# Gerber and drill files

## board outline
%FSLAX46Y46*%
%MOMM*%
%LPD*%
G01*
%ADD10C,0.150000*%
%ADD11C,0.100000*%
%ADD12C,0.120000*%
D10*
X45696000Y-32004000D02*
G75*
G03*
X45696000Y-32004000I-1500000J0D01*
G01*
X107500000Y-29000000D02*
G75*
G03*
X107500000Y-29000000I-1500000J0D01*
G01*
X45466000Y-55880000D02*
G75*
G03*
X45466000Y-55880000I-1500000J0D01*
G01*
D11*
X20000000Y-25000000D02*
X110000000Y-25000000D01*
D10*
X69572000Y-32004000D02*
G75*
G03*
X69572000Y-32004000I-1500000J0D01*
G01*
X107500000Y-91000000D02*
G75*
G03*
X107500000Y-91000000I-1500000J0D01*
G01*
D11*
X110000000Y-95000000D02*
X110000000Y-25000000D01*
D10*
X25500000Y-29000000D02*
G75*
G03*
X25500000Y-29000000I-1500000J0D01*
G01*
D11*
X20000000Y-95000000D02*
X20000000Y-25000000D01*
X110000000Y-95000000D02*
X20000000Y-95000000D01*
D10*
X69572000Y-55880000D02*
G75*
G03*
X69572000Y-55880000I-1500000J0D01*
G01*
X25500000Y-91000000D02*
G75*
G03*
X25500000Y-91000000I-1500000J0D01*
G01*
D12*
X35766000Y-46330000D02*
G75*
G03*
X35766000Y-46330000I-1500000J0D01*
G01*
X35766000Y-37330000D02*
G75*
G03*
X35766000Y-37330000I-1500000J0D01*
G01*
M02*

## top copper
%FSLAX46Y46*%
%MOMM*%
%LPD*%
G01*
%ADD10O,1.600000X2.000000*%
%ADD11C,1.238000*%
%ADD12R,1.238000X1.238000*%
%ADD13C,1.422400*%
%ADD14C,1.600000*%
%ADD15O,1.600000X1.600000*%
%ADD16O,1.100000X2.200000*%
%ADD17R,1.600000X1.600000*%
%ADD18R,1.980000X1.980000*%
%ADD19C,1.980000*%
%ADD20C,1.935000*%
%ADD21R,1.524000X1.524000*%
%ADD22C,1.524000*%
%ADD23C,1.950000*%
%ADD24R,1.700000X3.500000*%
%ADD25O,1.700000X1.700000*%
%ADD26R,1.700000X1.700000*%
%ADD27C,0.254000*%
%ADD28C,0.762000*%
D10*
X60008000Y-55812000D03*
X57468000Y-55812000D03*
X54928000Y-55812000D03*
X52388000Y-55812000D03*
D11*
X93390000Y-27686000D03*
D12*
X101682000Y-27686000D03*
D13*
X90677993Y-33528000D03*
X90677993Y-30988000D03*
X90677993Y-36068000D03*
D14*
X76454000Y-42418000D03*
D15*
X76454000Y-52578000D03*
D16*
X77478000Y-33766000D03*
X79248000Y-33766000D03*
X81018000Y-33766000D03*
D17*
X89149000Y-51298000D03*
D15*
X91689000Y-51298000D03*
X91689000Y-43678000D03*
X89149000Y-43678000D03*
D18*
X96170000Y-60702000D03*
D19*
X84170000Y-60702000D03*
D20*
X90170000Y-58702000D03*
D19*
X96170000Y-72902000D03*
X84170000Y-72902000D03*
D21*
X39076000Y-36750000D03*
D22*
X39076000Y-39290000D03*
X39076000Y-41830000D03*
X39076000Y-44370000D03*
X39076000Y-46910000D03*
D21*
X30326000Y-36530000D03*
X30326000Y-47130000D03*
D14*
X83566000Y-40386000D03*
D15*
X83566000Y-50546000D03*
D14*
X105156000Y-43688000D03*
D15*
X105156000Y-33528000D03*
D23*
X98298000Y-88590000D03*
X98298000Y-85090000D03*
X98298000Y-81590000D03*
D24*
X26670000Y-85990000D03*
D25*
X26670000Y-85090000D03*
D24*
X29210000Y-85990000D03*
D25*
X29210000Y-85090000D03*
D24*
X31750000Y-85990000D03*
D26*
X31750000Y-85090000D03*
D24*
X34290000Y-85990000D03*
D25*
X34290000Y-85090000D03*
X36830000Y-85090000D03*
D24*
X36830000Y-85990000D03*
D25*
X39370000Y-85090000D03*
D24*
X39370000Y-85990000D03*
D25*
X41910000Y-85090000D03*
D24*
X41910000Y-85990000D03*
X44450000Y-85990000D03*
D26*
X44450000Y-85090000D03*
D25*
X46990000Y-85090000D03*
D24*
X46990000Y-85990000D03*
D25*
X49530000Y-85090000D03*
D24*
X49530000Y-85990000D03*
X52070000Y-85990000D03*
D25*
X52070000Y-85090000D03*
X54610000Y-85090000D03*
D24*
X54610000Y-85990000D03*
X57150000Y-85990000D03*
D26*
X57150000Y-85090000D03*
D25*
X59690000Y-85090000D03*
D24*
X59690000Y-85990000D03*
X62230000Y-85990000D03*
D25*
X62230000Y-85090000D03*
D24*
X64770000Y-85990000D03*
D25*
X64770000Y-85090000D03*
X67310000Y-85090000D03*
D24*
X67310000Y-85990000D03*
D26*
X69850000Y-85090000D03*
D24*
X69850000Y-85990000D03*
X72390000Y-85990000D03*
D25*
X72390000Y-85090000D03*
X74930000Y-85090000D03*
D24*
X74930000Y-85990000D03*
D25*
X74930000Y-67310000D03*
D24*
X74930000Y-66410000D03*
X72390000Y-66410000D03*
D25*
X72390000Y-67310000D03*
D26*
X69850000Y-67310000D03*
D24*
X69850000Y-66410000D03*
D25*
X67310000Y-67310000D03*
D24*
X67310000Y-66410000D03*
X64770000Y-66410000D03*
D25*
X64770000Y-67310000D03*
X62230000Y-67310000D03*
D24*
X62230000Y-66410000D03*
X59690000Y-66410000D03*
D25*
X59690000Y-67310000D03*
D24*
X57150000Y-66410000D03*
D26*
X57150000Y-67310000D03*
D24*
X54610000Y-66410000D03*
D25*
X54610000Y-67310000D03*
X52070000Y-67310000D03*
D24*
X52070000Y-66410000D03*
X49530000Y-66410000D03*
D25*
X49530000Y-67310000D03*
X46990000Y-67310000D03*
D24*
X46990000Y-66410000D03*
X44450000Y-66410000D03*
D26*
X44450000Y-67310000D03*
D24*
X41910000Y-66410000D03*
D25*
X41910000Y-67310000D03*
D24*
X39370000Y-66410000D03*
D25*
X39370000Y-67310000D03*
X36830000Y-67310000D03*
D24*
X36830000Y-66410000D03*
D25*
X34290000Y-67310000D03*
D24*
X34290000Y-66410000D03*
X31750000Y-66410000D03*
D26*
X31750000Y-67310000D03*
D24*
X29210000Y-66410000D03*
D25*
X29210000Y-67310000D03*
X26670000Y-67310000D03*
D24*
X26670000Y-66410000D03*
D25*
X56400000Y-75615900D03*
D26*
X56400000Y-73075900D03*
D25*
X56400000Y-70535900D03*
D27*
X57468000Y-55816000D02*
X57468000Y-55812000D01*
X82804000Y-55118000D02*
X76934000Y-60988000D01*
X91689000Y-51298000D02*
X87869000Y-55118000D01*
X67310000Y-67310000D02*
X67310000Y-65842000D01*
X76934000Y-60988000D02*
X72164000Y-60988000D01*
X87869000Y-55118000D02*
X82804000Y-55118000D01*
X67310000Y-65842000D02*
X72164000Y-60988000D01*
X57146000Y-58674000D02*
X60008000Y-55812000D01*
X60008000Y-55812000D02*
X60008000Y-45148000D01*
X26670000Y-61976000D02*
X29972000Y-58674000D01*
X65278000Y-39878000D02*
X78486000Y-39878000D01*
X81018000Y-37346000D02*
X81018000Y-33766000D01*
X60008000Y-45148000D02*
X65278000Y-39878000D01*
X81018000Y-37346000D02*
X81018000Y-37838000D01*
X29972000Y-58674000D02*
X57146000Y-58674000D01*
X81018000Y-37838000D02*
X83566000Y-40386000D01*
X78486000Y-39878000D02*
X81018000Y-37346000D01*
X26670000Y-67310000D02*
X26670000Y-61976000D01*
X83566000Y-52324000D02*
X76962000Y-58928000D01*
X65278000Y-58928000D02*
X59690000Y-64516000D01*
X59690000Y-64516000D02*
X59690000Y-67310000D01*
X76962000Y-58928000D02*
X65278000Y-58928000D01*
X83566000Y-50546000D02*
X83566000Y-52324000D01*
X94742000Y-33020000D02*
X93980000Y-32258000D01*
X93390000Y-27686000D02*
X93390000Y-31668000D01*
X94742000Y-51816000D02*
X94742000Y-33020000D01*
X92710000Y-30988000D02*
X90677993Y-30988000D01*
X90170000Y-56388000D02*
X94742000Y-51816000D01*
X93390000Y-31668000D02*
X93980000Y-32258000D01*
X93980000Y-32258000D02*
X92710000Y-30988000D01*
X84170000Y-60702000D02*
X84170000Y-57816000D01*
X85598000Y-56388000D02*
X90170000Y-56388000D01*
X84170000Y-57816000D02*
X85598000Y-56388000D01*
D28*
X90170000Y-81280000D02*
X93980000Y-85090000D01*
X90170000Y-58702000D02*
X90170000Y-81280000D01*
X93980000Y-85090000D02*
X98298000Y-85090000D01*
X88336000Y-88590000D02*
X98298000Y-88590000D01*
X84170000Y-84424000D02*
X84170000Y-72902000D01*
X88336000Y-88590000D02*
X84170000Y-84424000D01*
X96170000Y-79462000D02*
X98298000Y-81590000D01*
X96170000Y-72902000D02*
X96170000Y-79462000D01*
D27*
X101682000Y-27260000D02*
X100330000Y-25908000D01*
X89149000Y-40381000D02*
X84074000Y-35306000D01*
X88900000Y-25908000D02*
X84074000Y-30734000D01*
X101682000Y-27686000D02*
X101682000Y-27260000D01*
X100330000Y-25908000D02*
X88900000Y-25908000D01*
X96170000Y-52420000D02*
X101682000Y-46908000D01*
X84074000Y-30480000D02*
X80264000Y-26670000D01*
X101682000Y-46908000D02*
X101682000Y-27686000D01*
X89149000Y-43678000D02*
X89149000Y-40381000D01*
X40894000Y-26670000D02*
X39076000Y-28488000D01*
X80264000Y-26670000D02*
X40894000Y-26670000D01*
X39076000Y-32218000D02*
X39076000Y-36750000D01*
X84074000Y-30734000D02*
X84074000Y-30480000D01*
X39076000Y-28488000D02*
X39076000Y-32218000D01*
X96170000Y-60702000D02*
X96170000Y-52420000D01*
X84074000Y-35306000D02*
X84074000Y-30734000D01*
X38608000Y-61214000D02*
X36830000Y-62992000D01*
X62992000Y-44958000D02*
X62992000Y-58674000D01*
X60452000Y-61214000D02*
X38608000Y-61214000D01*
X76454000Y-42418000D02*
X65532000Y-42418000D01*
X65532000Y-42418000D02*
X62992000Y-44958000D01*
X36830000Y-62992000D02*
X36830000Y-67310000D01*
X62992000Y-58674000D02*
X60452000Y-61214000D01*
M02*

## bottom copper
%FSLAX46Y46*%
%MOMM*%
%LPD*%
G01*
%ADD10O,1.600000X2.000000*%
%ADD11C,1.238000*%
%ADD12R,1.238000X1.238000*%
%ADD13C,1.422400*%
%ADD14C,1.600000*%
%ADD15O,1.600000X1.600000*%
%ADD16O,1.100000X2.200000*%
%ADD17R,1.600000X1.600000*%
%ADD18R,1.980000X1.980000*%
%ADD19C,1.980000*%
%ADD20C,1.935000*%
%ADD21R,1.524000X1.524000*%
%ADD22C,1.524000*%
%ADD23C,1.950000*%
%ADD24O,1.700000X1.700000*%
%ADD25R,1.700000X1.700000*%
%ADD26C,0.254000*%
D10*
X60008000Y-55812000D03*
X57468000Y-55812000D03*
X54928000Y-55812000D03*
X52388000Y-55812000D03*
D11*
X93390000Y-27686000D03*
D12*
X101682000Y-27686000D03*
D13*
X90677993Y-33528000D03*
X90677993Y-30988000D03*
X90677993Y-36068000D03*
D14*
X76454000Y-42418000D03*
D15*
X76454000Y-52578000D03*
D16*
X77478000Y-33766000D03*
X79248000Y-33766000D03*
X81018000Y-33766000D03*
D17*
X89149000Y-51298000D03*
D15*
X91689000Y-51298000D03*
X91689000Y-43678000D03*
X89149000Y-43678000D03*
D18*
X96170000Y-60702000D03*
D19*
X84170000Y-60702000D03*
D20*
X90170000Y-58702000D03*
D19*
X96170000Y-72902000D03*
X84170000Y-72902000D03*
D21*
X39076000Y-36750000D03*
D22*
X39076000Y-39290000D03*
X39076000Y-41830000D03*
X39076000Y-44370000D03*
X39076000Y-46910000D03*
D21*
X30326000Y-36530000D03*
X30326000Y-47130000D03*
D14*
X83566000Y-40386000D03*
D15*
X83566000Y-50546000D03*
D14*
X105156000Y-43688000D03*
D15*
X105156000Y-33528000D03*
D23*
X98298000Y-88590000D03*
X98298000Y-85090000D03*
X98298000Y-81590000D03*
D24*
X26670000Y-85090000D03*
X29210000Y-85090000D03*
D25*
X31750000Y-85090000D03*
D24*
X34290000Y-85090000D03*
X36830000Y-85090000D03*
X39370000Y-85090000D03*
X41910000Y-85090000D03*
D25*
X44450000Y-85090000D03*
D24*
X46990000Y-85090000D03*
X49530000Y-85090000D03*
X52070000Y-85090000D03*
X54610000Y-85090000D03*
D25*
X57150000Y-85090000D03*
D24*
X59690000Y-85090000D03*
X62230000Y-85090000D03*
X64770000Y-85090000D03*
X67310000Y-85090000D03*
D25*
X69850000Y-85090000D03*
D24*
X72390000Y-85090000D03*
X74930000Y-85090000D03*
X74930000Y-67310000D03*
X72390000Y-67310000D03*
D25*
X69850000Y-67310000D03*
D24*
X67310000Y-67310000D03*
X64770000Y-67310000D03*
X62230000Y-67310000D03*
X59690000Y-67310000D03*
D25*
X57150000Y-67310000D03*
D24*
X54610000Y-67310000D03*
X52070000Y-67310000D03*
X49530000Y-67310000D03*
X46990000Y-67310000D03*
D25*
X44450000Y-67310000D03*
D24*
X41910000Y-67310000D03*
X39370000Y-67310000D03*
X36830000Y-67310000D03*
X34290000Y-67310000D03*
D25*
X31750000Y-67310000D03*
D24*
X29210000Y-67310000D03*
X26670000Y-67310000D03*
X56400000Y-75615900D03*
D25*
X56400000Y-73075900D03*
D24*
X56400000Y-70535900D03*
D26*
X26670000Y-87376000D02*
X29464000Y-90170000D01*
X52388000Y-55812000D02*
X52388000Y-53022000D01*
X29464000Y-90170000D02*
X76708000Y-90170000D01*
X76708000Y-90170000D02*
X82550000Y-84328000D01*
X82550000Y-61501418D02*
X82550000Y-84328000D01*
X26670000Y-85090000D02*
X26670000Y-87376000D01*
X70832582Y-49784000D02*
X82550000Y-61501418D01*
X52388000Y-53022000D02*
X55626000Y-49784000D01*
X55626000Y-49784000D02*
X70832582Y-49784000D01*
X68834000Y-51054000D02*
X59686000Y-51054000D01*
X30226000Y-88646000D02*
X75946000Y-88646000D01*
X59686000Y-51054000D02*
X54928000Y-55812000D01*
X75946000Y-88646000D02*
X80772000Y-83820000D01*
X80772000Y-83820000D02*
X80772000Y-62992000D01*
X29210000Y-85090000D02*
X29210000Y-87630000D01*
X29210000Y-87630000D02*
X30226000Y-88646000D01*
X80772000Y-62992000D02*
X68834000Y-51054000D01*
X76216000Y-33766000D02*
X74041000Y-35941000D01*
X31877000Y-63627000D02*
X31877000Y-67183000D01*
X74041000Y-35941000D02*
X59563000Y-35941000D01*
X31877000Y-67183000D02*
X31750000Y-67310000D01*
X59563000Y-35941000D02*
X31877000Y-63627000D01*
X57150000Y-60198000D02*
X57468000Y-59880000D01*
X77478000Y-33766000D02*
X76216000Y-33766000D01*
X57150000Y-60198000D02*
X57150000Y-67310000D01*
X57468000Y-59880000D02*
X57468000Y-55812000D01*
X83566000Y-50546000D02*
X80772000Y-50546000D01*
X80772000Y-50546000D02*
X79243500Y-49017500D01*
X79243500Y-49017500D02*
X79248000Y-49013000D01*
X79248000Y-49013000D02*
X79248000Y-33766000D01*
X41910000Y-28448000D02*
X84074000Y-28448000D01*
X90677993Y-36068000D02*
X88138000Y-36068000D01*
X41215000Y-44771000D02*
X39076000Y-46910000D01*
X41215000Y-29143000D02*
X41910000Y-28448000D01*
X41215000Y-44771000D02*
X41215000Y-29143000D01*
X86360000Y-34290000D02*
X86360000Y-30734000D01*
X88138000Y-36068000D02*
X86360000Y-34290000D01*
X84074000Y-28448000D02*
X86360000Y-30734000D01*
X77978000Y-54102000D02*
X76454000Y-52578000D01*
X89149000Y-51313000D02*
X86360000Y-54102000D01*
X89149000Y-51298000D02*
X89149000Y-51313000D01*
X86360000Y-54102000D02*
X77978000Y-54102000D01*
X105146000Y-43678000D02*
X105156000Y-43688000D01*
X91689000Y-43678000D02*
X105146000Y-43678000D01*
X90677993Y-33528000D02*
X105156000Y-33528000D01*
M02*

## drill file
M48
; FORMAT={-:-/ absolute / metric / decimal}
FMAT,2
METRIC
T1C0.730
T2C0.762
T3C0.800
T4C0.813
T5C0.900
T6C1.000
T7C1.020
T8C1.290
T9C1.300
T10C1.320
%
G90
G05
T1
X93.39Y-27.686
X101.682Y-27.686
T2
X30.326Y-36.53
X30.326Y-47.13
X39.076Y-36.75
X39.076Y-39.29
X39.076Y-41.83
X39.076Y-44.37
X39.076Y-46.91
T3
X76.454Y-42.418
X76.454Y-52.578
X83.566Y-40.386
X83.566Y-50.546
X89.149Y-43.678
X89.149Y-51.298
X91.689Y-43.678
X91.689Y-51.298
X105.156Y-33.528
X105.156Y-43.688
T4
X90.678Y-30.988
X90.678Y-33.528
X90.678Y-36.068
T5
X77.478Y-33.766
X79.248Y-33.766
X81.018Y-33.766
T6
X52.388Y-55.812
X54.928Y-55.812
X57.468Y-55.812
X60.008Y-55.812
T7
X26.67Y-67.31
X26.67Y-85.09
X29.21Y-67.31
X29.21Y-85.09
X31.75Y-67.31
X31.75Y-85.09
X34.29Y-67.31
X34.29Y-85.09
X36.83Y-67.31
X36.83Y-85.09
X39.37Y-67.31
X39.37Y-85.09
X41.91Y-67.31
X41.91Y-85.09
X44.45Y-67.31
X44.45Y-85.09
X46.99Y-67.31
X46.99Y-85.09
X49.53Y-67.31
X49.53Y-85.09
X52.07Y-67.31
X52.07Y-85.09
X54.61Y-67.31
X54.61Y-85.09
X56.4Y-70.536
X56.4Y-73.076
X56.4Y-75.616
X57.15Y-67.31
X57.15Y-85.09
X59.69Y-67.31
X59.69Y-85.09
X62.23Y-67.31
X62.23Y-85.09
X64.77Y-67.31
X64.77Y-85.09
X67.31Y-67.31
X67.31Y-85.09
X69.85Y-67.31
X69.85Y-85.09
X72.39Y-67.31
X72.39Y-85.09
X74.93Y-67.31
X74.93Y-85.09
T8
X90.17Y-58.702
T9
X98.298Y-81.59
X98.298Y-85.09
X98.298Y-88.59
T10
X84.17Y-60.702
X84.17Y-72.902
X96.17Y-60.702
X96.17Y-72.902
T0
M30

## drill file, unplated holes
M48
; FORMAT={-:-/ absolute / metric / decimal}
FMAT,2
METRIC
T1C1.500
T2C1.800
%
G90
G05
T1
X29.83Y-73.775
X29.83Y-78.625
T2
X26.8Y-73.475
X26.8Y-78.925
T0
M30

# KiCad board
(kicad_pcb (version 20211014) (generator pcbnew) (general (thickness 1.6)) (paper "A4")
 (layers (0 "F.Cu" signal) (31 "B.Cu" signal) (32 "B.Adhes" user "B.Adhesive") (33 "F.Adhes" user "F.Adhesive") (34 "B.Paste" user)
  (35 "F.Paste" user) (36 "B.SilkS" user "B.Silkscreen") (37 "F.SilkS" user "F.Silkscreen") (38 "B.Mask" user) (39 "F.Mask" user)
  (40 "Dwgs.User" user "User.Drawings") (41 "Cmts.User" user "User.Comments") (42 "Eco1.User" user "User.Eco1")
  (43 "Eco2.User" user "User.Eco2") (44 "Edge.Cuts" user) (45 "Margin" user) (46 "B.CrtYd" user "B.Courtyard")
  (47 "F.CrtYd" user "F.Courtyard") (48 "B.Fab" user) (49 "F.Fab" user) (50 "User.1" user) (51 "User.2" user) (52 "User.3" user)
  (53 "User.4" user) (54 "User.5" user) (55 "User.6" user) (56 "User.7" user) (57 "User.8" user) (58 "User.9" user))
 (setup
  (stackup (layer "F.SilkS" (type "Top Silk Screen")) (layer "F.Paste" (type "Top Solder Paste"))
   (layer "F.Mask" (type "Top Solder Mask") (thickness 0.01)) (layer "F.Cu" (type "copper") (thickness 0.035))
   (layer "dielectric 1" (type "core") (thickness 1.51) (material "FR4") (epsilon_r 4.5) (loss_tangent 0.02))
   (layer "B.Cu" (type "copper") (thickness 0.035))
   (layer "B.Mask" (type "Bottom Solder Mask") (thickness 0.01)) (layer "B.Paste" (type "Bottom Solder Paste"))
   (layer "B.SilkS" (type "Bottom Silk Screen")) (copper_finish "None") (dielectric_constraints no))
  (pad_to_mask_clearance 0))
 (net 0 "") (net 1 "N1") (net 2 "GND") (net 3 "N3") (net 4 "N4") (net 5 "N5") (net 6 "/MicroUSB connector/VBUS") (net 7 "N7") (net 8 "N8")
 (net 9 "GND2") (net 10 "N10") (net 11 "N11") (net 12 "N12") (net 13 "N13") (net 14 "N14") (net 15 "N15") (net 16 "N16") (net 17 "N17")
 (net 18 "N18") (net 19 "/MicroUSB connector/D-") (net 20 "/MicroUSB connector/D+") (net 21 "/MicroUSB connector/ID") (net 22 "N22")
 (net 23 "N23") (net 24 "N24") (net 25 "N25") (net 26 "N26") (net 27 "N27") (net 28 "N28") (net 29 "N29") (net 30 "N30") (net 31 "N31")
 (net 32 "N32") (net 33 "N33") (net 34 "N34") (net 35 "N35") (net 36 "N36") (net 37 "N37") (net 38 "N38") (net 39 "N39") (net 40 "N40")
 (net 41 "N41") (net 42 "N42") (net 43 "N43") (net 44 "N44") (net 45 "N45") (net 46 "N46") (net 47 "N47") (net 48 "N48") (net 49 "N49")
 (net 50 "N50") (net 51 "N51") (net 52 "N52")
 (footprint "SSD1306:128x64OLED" (layer "F.Cu") (at 56.388 45.212 180)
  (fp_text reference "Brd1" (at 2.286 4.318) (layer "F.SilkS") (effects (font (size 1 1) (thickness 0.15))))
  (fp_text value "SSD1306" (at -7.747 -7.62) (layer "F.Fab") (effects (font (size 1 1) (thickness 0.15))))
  (pad "1" thru_hole oval locked (at -3.62 -10.6 270) (size 2 1.6) (drill 1) (layers *.Cu *.Mask) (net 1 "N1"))
  (pad "2" thru_hole oval locked (at -1.08 -10.6 270) (size 2 1.6) (drill 1) (layers *.Cu *.Mask) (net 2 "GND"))
  (pad "3" thru_hole oval locked (at 1.46 -10.6 270) (size 2 1.6) (drill 1) (layers *.Cu *.Mask) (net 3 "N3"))
  (pad "4" thru_hole oval locked (at 4 -10.6 270) (size 2 1.6) (drill 1) (layers *.Cu *.Mask) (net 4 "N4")))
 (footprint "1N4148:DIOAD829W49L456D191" (layer "F.Cu") (at 97.536 27.686 180)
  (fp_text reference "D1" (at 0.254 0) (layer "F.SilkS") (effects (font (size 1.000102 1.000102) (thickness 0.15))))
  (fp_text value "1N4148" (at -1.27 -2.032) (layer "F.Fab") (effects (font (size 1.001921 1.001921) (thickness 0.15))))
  (pad "A" thru_hole circle locked (at 4.146 0 180) (size 1.238 1.238) (drill 0.73) (layers *.Cu *.Mask) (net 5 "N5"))
  (pad "C" thru_hole rect locked (at -4.146 0 180) (size 1.238 1.238) (drill 0.73) (layers *.Cu *.Mask) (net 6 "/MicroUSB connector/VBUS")))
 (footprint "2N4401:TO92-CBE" (layer "F.Cu") (at 90.677993 33.528 90)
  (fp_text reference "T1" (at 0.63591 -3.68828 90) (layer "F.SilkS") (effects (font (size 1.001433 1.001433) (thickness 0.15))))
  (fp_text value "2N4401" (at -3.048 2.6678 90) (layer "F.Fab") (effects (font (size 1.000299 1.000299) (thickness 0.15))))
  (pad "B" thru_hole circle locked (at 0 0 90) (size 1.4224 1.4224) (drill 0.8128) (layers *.Cu *.Mask) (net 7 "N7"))
  (pad "C" thru_hole circle locked (at 2.54 0 90) (size 1.4224 1.4224) (drill 0.8128) (layers *.Cu *.Mask) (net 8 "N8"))
  (pad "E" thru_hole circle locked (at -2.54 0 90) (size 1.4224 1.4224) (drill 0.8128) (layers *.Cu *.Mask) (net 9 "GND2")))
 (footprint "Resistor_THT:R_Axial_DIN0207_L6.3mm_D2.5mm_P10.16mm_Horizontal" (layer "F.Cu") (at 76.454 42.418 -90)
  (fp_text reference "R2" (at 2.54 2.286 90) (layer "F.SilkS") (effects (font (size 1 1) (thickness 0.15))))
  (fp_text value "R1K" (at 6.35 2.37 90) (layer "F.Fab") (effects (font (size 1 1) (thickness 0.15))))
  (pad "1" thru_hole circle (at 0 0 270) (size 1.6 1.6) (drill 0.8) (layers *.Cu *.Mask) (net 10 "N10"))
  (pad "2" thru_hole oval (at 10.16 0 270) (size 1.6 1.6) (drill 0.8) (layers *.Cu *.Mask) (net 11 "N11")))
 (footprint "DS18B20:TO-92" (layer "F.Cu") (at 79.248 32.766)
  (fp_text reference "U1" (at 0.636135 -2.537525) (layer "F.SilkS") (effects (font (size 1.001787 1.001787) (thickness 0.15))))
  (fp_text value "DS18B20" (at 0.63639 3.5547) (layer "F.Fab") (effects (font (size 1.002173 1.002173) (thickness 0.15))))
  (pad "1" thru_hole oval locked (at -1.77 1) (size 1.1 2.2) (drill 0.9) (layers *.Cu *.Mask) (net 2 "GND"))
  (pad "2" thru_hole oval locked (at 0 1) (size 1.1 2.2) (drill 0.9) (layers *.Cu *.Mask) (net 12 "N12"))
  (pad "3" thru_hole oval locked (at 1.77 1) (size 1.1 2.2) (drill 0.9) (layers *.Cu *.Mask) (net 1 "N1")))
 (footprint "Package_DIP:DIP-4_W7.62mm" (layer "F.Cu") (at 89.149 51.298 90)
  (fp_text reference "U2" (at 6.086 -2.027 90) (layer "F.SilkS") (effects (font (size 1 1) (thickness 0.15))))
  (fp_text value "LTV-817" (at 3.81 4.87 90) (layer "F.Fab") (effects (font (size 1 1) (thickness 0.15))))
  (pad "1" thru_hole rect (at 0 0 90) (size 1.6 1.6) (drill 0.8) (layers *.Cu *.Mask) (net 11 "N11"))
  (pad "2" thru_hole oval (at 0 2.54 90) (size 1.6 1.6) (drill 0.8) (layers *.Cu *.Mask) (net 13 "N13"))
  (pad "3" thru_hole oval (at 7.62 2.54 90) (size 1.6 1.6) (drill 0.8) (layers *.Cu *.Mask) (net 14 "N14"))
  (pad "4" thru_hole oval (at 7.62 0 90) (size 1.6 1.6) (drill 0.8) (layers *.Cu *.Mask) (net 6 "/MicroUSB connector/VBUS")))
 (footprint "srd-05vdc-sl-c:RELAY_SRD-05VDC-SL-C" (layer "F.Cu") (at 90.17 66.802 -90)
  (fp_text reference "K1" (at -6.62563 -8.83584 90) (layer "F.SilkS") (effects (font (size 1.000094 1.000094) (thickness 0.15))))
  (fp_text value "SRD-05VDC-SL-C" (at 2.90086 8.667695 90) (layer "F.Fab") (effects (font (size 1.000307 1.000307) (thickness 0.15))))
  (pad "A1" thru_hole rect locked (at -6.1 -6 270) (size 1.98 1.98) (drill 1.32) (layers *.Cu *.Mask) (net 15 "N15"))
  (pad "A2" thru_hole circle locked (at -6.1 6 270) (size 1.98 1.98) (drill 1.32) (layers *.Cu *.Mask) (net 8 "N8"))
  (pad "COM" thru_hole circle locked (at -8.1 0 270) (size 1.935 1.935) (drill 1.29) (layers *.Cu *.Mask) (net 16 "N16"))
  (pad "NC" thru_hole circle locked (at 6.1 -6 270) (size 1.98 1.98) (drill 1.32) (layers *.Cu *.Mask) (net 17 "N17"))
  (pad "NO" thru_hole circle locked (at 6.1 6 270) (size 1.98 1.98) (drill 1.32) (layers *.Cu *.Mask) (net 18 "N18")))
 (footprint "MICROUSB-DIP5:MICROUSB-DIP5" (layer "F.Cu") (at 32.766 41.83)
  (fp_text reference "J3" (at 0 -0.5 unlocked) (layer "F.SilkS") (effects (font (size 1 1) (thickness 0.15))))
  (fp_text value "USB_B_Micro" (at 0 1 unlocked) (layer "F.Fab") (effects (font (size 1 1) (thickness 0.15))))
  (fp_circle (center 1.5 4.5) (end 3 4.5) (layer "Edge.Cuts") (width 0.12) (fill none))
  (fp_circle (center 1.5 -4.5) (end 3 -4.5) (layer "Edge.Cuts") (width 0.12) (fill none))
  (pad "1" thru_hole rect (at 6.31 -5.08) (size 1.524 1.524) (drill 0.762) (layers *.Cu *.Mask) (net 6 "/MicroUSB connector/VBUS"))
  (pad "2" thru_hole circle (at 6.31 -2.54) (size 1.524 1.524) (drill 0.762) (layers *.Cu *.Mask) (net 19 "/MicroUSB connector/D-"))
  (pad "3" thru_hole circle (at 6.31 0) (size 1.524 1.524) (drill 0.762) (layers *.Cu *.Mask) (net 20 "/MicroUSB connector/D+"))
  (pad "4" thru_hole circle (at 6.31 2.54) (size 1.524 1.524) (drill 0.762) (layers *.Cu *.Mask) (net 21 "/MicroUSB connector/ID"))
  (pad "5" thru_hole circle (at 6.31 5.08) (size 1.524 1.524) (drill 0.762) (layers *.Cu *.Mask) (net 9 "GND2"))
  (pad "6" thru_hole rect (at -2.44 -5.3) (size 1.524 1.524) (drill 0.762) (layers *.Cu *.Mask) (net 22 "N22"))
  (pad "7" thru_hole rect (at -2.44 5.3) (size 1.524 1.524) (drill 0.762) (layers *.Cu *.Mask)))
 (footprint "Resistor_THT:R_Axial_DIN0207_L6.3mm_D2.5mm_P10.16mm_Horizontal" (layer "F.Cu") (at 83.566 40.386 -90)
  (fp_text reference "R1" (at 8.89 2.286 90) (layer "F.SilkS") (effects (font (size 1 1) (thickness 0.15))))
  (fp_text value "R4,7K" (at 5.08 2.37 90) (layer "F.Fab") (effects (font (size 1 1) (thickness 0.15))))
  (pad "1" thru_hole circle (at 0 0 270) (size 1.6 1.6) (drill 0.8) (layers *.Cu *.Mask) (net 1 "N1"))
  (pad "2" thru_hole oval (at 10.16 0 270) (size 1.6 1.6) (drill 0.8) (layers *.Cu *.Mask) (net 12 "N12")))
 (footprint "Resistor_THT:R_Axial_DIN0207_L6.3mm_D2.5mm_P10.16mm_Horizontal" (layer "F.Cu") (at 105.156 43.688 90)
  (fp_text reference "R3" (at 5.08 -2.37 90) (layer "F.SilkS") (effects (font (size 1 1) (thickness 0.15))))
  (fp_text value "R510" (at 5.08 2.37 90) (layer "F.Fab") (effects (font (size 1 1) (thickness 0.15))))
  (pad "1" thru_hole circle (at 0 0 90) (size 1.6 1.6) (drill 0.8) (layers *.Cu *.Mask) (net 14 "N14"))
  (pad "2" thru_hole oval (at 10.16 0 90) (size 1.6 1.6) (drill 0.8) (layers *.Cu *.Mask) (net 7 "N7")))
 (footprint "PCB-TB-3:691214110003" (layer "F.Cu") (at 98.298 85.09 90)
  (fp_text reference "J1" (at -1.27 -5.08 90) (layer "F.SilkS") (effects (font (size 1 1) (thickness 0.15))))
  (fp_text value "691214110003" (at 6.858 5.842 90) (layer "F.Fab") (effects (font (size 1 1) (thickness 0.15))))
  (pad "1" thru_hole circle locked (at -3.5 0 90) (size 1.95 1.95) (drill 1.3) (layers *.Cu *.Mask) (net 18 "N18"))
  (pad "2" thru_hole circle locked (at 0 0 90) (size 1.95 1.95) (drill 1.3) (layers *.Cu *.Mask) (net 16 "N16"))
  (pad "3" thru_hole circle locked (at 3.5 0 90) (size 1.95 1.95) (drill 1.3) (layers *.Cu *.Mask) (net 17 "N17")))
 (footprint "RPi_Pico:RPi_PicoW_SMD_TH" (layer "F.Cu") (at 50.8 76.2 90)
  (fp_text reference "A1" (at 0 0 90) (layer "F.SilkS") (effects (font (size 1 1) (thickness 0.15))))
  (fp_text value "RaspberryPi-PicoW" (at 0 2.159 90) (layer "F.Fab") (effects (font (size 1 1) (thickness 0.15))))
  (pad "" np_thru_hole oval (at -2.425 -20.97 90) (size 1.5 1.5) (drill 1.5) (layers *.Cu *.Mask))
  (pad "" np_thru_hole oval (at 2.725 -24 90) (size 1.8 1.8) (drill 1.8) (layers *.Cu *.Mask))
  (pad "" np_thru_hole oval (at 2.425 -20.97 90) (size 1.5 1.5) (drill 1.5) (layers *.Cu *.Mask))
  (pad "" np_thru_hole oval (at -2.725 -24 90) (size 1.8 1.8) (drill 1.8) (layers *.Cu *.Mask))
  (pad "1" smd rect (at -8.89 -24.13 90) (size 3.5 1.7) (drill (offset -0.9 0)) (layers "F.Cu" "F.Mask") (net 4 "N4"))
  (pad "1" thru_hole oval (at -8.89 -24.13 90) (size 1.7 1.7) (drill 1.02) (layers *.Cu *.Mask) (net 4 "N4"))
  (pad "2" smd rect (at -8.89 -21.59 90) (size 3.5 1.7) (drill (offset -0.9 0)) (layers "F.Cu" "F.Mask") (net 3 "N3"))
  (pad "2" thru_hole oval (at -8.89 -21.59 90) (size 1.7 1.7) (drill 1.02) (layers *.Cu *.Mask) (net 3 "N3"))
  (pad "3" smd rect (at -8.89 -19.05 90) (size 3.5 1.7) (drill (offset -0.9 0)) (layers "F.Cu" "F.Mask") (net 2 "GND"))
  (pad "3" thru_hole rect (at -8.89 -19.05 90) (size 1.7 1.7) (drill 1.02) (layers *.Cu *.Mask) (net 2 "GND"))
  (pad "4" smd rect (at -8.89 -16.51 90) (size 3.5 1.7) (drill (offset -0.9 0)) (layers "F.Cu" "F.Mask") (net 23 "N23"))
  (pad "4" thru_hole oval (at -8.89 -16.51 90) (size 1.7 1.7) (drill 1.02) (layers *.Cu *.Mask) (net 23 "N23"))
  (pad "5" thru_hole oval (at -8.89 -13.97 90) (size 1.7 1.7) (drill 1.02) (layers *.Cu *.Mask) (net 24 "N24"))
  (pad "5" smd rect (at -8.89 -13.97 90) (size 3.5 1.7) (drill (offset -0.9 0)) (layers "F.Cu" "F.Mask") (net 24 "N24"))
  (pad "6" thru_hole oval (at -8.89 -11.43 90) (size 1.7 1.7) (drill 1.02) (layers *.Cu *.Mask) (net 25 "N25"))
  (pad "6" smd rect (at -8.89 -11.43 90) (size 3.5 1.7) (drill (offset -0.9 0)) (layers "F.Cu" "F.Mask") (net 25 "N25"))
  (pad "7" thru_hole oval (at -8.89 -8.89 90) (size 1.7 1.7) (drill 1.02) (layers *.Cu *.Mask) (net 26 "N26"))
  (pad "7" smd rect (at -8.89 -8.89 90) (size 3.5 1.7) (drill (offset -0.9 0)) (layers "F.Cu" "F.Mask") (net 26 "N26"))
  (pad "8" smd rect (at -8.89 -6.35 90) (size 3.5 1.7) (drill (offset -0.9 0)) (layers "F.Cu" "F.Mask") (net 2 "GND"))
  (pad "8" thru_hole rect (at -8.89 -6.35 90) (size 1.7 1.7) (drill 1.02) (layers *.Cu *.Mask) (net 2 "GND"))
  (pad "9" thru_hole oval (at -8.89 -3.81 90) (size 1.7 1.7) (drill 1.02) (layers *.Cu *.Mask) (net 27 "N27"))
  (pad "9" smd rect (at -8.89 -3.81 90) (size 3.5 1.7) (drill (offset -0.9 0)) (layers "F.Cu" "F.Mask") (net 27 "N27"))
  (pad "10" thru_hole oval (at -8.89 -1.27 90) (size 1.7 1.7) (drill 1.02) (layers *.Cu *.Mask) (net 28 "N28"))
  (pad "10" smd rect (at -8.89 -1.27 90) (size 3.5 1.7) (drill (offset -0.9 0)) (layers "F.Cu" "F.Mask") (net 28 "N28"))
  (pad "11" smd rect (at -8.89 1.27 90) (size 3.5 1.7) (drill (offset -0.9 0)) (layers "F.Cu" "F.Mask") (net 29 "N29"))
  (pad "11" thru_hole oval (at -8.89 1.27 90) (size 1.7 1.7) (drill 1.02) (layers *.Cu *.Mask) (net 29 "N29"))
  (pad "12" thru_hole oval (at -8.89 3.81 90) (size 1.7 1.7) (drill 1.02) (layers *.Cu *.Mask) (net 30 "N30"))
  (pad "12" smd rect (at -8.89 3.81 90) (size 3.5 1.7) (drill (offset -0.9 0)) (layers "F.Cu" "F.Mask") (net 30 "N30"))
  (pad "13" smd rect (at -8.89 6.35 90) (size 3.5 1.7) (drill (offset -0.9 0)) (layers "F.Cu" "F.Mask") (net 2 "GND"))
  (pad "13" thru_hole rect (at -8.89 6.35 90) (size 1.7 1.7) (drill 1.02) (layers *.Cu *.Mask) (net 2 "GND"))
  (pad "14" thru_hole oval (at -8.89 8.89 90) (size 1.7 1.7) (drill 1.02) (layers *.Cu *.Mask) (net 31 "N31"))
  (pad "14" smd rect (at -8.89 8.89 90) (size 3.5 1.7) (drill (offset -0.9 0)) (layers "F.Cu" "F.Mask") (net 31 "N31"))
  (pad "15" smd rect (at -8.89 11.43 90) (size 3.5 1.7) (drill (offset -0.9 0)) (layers "F.Cu" "F.Mask") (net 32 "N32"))
  (pad "15" thru_hole oval (at -8.89 11.43 90) (size 1.7 1.7) (drill 1.02) (layers *.Cu *.Mask) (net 32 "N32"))
  (pad "16" smd rect (at -8.89 13.97 90) (size 3.5 1.7) (drill (offset -0.9 0)) (layers "F.Cu" "F.Mask") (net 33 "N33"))
  (pad "16" thru_hole oval (at -8.89 13.97 90) (size 1.7 1.7) (drill 1.02) (layers *.Cu *.Mask) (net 33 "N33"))
  (pad "17" thru_hole oval (at -8.89 16.51 90) (size 1.7 1.7) (drill 1.02) (layers *.Cu *.Mask) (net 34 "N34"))
  (pad "17" smd rect (at -8.89 16.51 90) (size 3.5 1.7) (drill (offset -0.9 0)) (layers "F.Cu" "F.Mask") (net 34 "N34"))
  (pad "18" thru_hole rect (at -8.89 19.05 90) (size 1.7 1.7) (drill 1.02) (layers *.Cu *.Mask) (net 2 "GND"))
  (pad "18" smd rect (at -8.89 19.05 90) (size 3.5 1.7) (drill (offset -0.9 0)) (layers "F.Cu" "F.Mask") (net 2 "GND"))
  (pad "19" smd rect (at -8.89 21.59 90) (size 3.5 1.7) (drill (offset -0.9 0)) (layers "F.Cu" "F.Mask") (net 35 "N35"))
  (pad "19" thru_hole oval (at -8.89 21.59 90) (size 1.7 1.7) (drill 1.02) (layers *.Cu *.Mask) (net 35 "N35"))
  (pad "20" thru_hole oval (at -8.89 24.13 90) (size 1.7 1.7) (drill 1.02) (layers *.Cu *.Mask) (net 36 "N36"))
  (pad "20" smd rect (at -8.89 24.13 90) (size 3.5 1.7) (drill (offset -0.9 0)) (layers "F.Cu" "F.Mask") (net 36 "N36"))
  (pad "21" thru_hole oval (at 8.89 24.13 90) (size 1.7 1.7) (drill 1.02) (layers *.Cu *.Mask) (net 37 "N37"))
  (pad "21" smd rect (at 8.89 24.13 90) (size 3.5 1.7) (drill (offset 0.9 0)) (layers "F.Cu" "F.Mask") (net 37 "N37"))
  (pad "22" smd rect (at 8.89 21.59 90) (size 3.5 1.7) (drill (offset 0.9 0)) (layers "F.Cu" "F.Mask") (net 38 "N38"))
  (pad "22" thru_hole oval (at 8.89 21.59 90) (size 1.7 1.7) (drill 1.02) (layers *.Cu *.Mask) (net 38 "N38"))
  (pad "23" thru_hole rect (at 8.89 19.05 90) (size 1.7 1.7) (drill 1.02) (layers *.Cu *.Mask) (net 2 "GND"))
  (pad "23" smd rect (at 8.89 19.05 90) (size 3.5 1.7) (drill (offset 0.9 0)) (layers "F.Cu" "F.Mask") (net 2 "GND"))
  (pad "24" thru_hole oval (at 8.89 16.51 90) (size 1.7 1.7) (drill 1.02) (layers *.Cu *.Mask) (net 13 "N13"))
  (pad "24" smd rect (at 8.89 16.51 90) (size 3.5 1.7) (drill (offset 0.9 0)) (layers "F.Cu" "F.Mask") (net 13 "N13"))
  (pad "25" smd rect (at 8.89 13.97 90) (size 3.5 1.7) (drill (offset 0.9 0)) (layers "F.Cu" "F.Mask") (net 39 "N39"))
  (pad "25" thru_hole oval (at 8.89 13.97 90) (size 1.7 1.7) (drill 1.02) (layers *.Cu *.Mask) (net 39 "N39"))
  (pad "26" thru_hole oval (at 8.89 11.43 90) (size 1.7 1.7) (drill 1.02) (layers *.Cu *.Mask) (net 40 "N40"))
  (pad "26" smd rect (at 8.89 11.43 90) (size 3.5 1.7) (drill (offset 0.9 0)) (layers "F.Cu" "F.Mask") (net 40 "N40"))
  (pad "27" smd rect (at 8.89 8.89 90) (size 3.5 1.7) (drill (offset 0.9 0)) (layers "F.Cu" "F.Mask") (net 12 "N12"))
  (pad "27" thru_hole oval (at 8.89 8.89 90) (size 1.7 1.7) (drill 1.02) (layers *.Cu *.Mask) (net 12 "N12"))
  (pad "28" smd rect (at 8.89 6.35 90) (size 3.5 1.7) (drill (offset 0.9 0)) (layers "F.Cu" "F.Mask") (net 2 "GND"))
  (pad "28" thru_hole rect (at 8.89 6.35 90) (size 1.7 1.7) (drill 1.02) (layers *.Cu *.Mask) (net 2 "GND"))
  (pad "29" smd rect (at 8.89 3.81 90) (size 3.5 1.7) (drill (offset 0.9 0)) (layers "F.Cu" "F.Mask") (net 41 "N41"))
  (pad "29" thru_hole oval (at 8.89 3.81 90) (size 1.7 1.7) (drill 1.02) (layers *.Cu *.Mask) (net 41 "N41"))
  (pad "30" thru_hole oval (at 8.89 1.27 90) (size 1.7 1.7) (drill 1.02) (layers *.Cu *.Mask) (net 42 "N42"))
  (pad "30" smd rect (at 8.89 1.27 90) (size 3.5 1.7) (drill (offset 0.9 0)) (layers "F.Cu" "F.Mask") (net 42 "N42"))
  (pad "31" smd rect (at 8.89 -1.27 90) (size 3.5 1.7) (drill (offset 0.9 0)) (layers "F.Cu" "F.Mask") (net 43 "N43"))
  (pad "31" thru_hole oval (at 8.89 -1.27 90) (size 1.7 1.7) (drill 1.02) (layers *.Cu *.Mask) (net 43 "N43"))
  (pad "32" thru_hole oval (at 8.89 -3.81 90) (size 1.7 1.7) (drill 1.02) (layers *.Cu *.Mask) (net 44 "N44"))
  (pad "32" smd rect (at 8.89 -3.81 90) (size 3.5 1.7) (drill (offset 0.9 0)) (layers "F.Cu" "F.Mask") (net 44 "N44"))
  (pad "33" smd rect (at 8.89 -6.35 90) (size 3.5 1.7) (drill (offset 0.9 0)) (layers "F.Cu" "F.Mask") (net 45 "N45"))
  (pad "33" thru_hole rect (at 8.89 -6.35 90) (size 1.7 1.7) (drill 1.02) (layers *.Cu *.Mask) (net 45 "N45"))
  (pad "34" smd rect (at 8.89 -8.89 90) (size 3.5 1.7) (drill (offset 0.9 0)) (layers "F.Cu" "F.Mask") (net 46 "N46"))
  (pad "34" thru_hole oval (at 8.89 -8.89 90) (size 1.7 1.7) (drill 1.02) (layers *.Cu *.Mask) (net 46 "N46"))
  (pad "35" smd rect (at 8.89 -11.43 90) (size 3.5 1.7) (drill (offset 0.9 0)) (layers "F.Cu" "F.Mask") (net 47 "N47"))
  (pad "35" thru_hole oval (at 8.89 -11.43 90) (size 1.7 1.7) (drill 1.02) (layers *.Cu *.Mask) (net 47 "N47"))
  (pad "36" thru_hole oval (at 8.89 -13.97 90) (size 1.7 1.7) (drill 1.02) (layers *.Cu *.Mask) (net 10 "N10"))
  (pad "36" smd rect (at 8.89 -13.97 90) (size 3.5 1.7) (drill (offset 0.9 0)) (layers "F.Cu" "F.Mask") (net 10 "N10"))
  (pad "37" thru_hole oval (at 8.89 -16.51 90) (size 1.7 1.7) (drill 1.02) (layers *.Cu *.Mask) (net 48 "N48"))
  (pad "37" smd rect (at 8.89 -16.51 90) (size 3.5 1.7) (drill (offset 0.9 0)) (layers "F.Cu" "F.Mask") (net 48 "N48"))
  (pad "38" smd rect (at 8.89 -19.05 90) (size 3.5 1.7) (drill (offset 0.9 0)) (layers "F.Cu" "F.Mask") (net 2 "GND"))
  (pad "38" thru_hole rect (at 8.89 -19.05 90) (size 1.7 1.7) (drill 1.02) (layers *.Cu *.Mask) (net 2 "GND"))
  (pad "39" smd rect (at 8.89 -21.59 90) (size 3.5 1.7) (drill (offset 0.9 0)) (layers "F.Cu" "F.Mask") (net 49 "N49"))
  (pad "39" thru_hole oval (at 8.89 -21.59 90) (size 1.7 1.7) (drill 1.02) (layers *.Cu *.Mask) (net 49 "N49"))
  (pad "40" thru_hole oval (at 8.89 -24.13 90) (size 1.7 1.7) (drill 1.02) (layers *.Cu *.Mask) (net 1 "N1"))
  (pad "40" smd rect (at 8.89 -24.13 90) (size 3.5 1.7) (drill (offset 0.9 0)) (layers "F.Cu" "F.Mask") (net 1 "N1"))
  (pad "41" thru_hole oval (at 0.5841 5.6 90) (size 1.7 1.7) (drill 1.02) (layers *.Cu *.Mask) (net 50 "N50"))
  (pad "42" thru_hole rect (at 3.1241 5.6 90) (size 1.7 1.7) (drill 1.02) (layers *.Cu *.Mask) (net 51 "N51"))
  (pad "43" thru_hole oval (at 5.6641 5.6 90) (size 1.7 1.7) (drill 1.02) (layers *.Cu *.Mask) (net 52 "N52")))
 (gr_circle (center 44.196 32.004) (end 45.696 32.004) (layer "Edge.Cuts") (width 0.15) (fill none))
 (gr_circle (center 106 29) (end 107.5 29) (layer "Edge.Cuts") (width 0.15) (fill none))
 (gr_circle (center 43.966 55.88) (end 45.466 55.88) (layer "Edge.Cuts") (width 0.15) (fill none))
 (gr_line (start 20 25) (end 110 25) (layer "Edge.Cuts") (width 0.1))
 (gr_circle (center 68.072 32.004) (end 69.572 32.004) (layer "Edge.Cuts") (width 0.15) (fill none))
 (gr_circle (center 106 91) (end 107.5 91) (layer "Edge.Cuts") (width 0.15) (fill none))
 (gr_line (start 110 95) (end 110 25) (layer "Edge.Cuts") (width 0.1))
 (gr_circle (center 24 29) (end 25.5 29) (layer "Edge.Cuts") (width 0.15) (fill none))
 (gr_line (start 20 95) (end 20 25) (layer "Edge.Cuts") (width 0.1))
 (gr_line (start 110 95) (end 20 95) (layer "Edge.Cuts") (width 0.1))
 (gr_circle (center 68.072 55.88) (end 69.572 55.88) (layer "Edge.Cuts") (width 0.15) (fill none))
 (gr_circle (center 24 91) (end 25.5 91) (layer "Edge.Cuts") (width 0.15) (fill none))
 (segment (start 26.67 87.376) (end 29.464 90.17) (width 0.254) (layer "B.Cu") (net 4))
 (segment (start 52.388 55.812) (end 52.388 53.022) (width 0.254) (layer "B.Cu") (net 4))
 (segment (start 29.464 90.17) (end 76.708 90.17) (width 0.254) (layer "B.Cu") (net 4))
 (segment (start 76.708 90.17) (end 82.55 84.328) (width 0.254) (layer "B.Cu") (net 4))
 (segment (start 82.55 61.501418) (end 82.55 84.328) (width 0.254) (layer "B.Cu") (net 4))
 (segment (start 26.67 85.09) (end 26.67 87.376) (width 0.254) (layer "B.Cu") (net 4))
 (segment (start 70.832582 49.784) (end 82.55 61.501418) (width 0.254) (layer "B.Cu") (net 4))
 (segment (start 52.388 53.022) (end 55.626 49.784) (width 0.254) (layer "B.Cu") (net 4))
 (segment (start 55.626 49.784) (end 70.832582 49.784) (width 0.254) (layer "B.Cu") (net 4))
 (segment (start 68.834 51.054) (end 59.686 51.054) (width 0.254) (layer "B.Cu") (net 3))
 (segment (start 30.226 88.646) (end 75.946 88.646) (width 0.254) (layer "B.Cu") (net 3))
 (segment (start 59.686 51.054) (end 54.928 55.812) (width 0.254) (layer "B.Cu") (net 3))
 (segment (start 75.946 88.646) (end 80.772 83.82) (width 0.254) (layer "B.Cu") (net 3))
 (segment (start 80.772 83.82) (end 80.772 62.992) (width 0.254) (layer "B.Cu") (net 3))
 (segment (start 29.21 85.09) (end 29.21 87.63) (width 0.254) (layer "B.Cu") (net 3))
 (segment (start 29.21 87.63) (end 30.226 88.646) (width 0.254) (layer "B.Cu") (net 3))
 (segment (start 80.772 62.992) (end 68.834 51.054) (width 0.254) (layer "B.Cu") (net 3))
 (segment (start 57.468 55.816) (end 57.468 55.812) (width 0.254) (layer "F.Cu") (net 2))
 (segment (start 76.216 33.766) (end 74.041 35.941) (width 0.254) (layer "B.Cu") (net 2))
 (segment (start 31.877 63.627) (end 31.877 67.183) (width 0.254) (layer "B.Cu") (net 2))
 (segment (start 74.041 35.941) (end 59.563 35.941) (width 0.254) (layer "B.Cu") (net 2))
 (segment (start 31.877 67.183) (end 31.75 67.31) (width 0.254) (layer "B.Cu") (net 2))
 (segment (start 59.563 35.941) (end 31.877 63.627) (width 0.254) (layer "B.Cu") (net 2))
 (segment (start 57.15 60.198) (end 57.468 59.88) (width 0.254) (layer "B.Cu") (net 2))
 (segment (start 77.478 33.766) (end 76.216 33.766) (width 0.254) (layer "B.Cu") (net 2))
 (segment (start 57.15 60.198) (end 57.15 67.31) (width 0.254) (layer "B.Cu") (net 2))
 (segment (start 57.468 59.88) (end 57.468 55.812) (width 0.254) (layer "B.Cu") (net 2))
 (segment (start 82.804 55.118) (end 76.934 60.988) (width 0.254) (layer "F.Cu") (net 13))
 (segment (start 91.689 51.298) (end 87.869 55.118) (width 0.254) (layer "F.Cu") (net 13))
 (segment (start 67.31 67.31) (end 67.31 65.842) (width 0.254) (layer "F.Cu") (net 13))
 (segment (start 76.934 60.988) (end 72.164 60.988) (width 0.254) (layer "F.Cu") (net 13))
 (segment (start 87.869 55.118) (end 82.804 55.118) (width 0.254) (layer "F.Cu") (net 13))
 (segment (start 67.31 65.842) (end 72.164 60.988) (width 0.254) (layer "F.Cu") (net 13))
 (segment (start 57.146 58.674) (end 60.008 55.812) (width 0.254) (layer "F.Cu") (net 1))
 (segment (start 60.008 55.812) (end 60.008 45.148) (width 0.254) (layer "F.Cu") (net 1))
 (segment (start 26.67 61.976) (end 29.972 58.674) (width 0.254) (layer "F.Cu") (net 1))
 (segment (start 65.278 39.878) (end 78.486 39.878) (width 0.254) (layer "F.Cu") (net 1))
 (segment (start 81.018 37.346) (end 81.018 33.766) (width 0.254) (layer "F.Cu") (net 1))
 (segment (start 60.008 45.148) (end 65.278 39.878) (width 0.254) (layer "F.Cu") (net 1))
 (segment (start 81.018 37.346) (end 81.018 37.838) (width 0.254) (layer "F.Cu") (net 1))
 (segment (start 29.972 58.674) (end 57.146 58.674) (width 0.254) (layer "F.Cu") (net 1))
 (segment (start 81.018 37.838) (end 83.566 40.386) (width 0.254) (layer "F.Cu") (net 1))
 (segment (start 78.486 39.878) (end 81.018 37.346) (width 0.254) (layer "F.Cu") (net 1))
 (segment (start 26.67 67.31) (end 26.67 61.976) (width 0.254) (layer "F.Cu") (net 1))
 (segment (start 83.566 52.324) (end 76.962 58.928) (width 0.254) (layer "F.Cu") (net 12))
 (segment (start 65.278 58.928) (end 59.69 64.516) (width 0.254) (layer "F.Cu") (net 12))
 (segment (start 59.69 64.516) (end 59.69 67.31) (width 0.254) (layer "F.Cu") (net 12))
 (segment (start 76.962 58.928) (end 65.278 58.928) (width 0.254) (layer "F.Cu") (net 12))
 (segment (start 83.566 50.546) (end 83.566 52.324) (width 0.254) (layer "F.Cu") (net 12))
 (segment (start 83.566 50.546) (end 80.772 50.546) (width 0.254) (layer "B.Cu") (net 12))
 (segment (start 80.772 50.546) (end 79.2435 49.0175) (width 0.254) (layer "B.Cu") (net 12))
 (segment (start 79.2435 49.0175) (end 79.248 49.013) (width 0.254) (layer "B.Cu") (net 12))
 (segment (start 79.248 49.013) (end 79.248 33.766) (width 0.254) (layer "B.Cu") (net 12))
 (segment (start 41.91 28.448) (end 84.074 28.448) (width 0.254) (layer "B.Cu") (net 9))
 (segment (start 90.677993 36.068) (end 88.138 36.068) (width 0.254) (layer "B.Cu") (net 9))
 (segment (start 41.215 44.771) (end 39.076 46.91) (width 0.254) (layer "B.Cu") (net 9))
 (segment (start 41.215 29.143) (end 41.91 28.448) (width 0.254) (layer "B.Cu") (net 9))
 (segment (start 41.215 44.771) (end 41.215 29.143) (width 0.254) (layer "B.Cu") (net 9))
 (segment (start 86.36 34.29) (end 86.36 30.734) (width 0.254) (layer "B.Cu") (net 9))
 (segment (start 88.138 36.068) (end 86.36 34.29) (width 0.254) (layer "B.Cu") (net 9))
 (segment (start 84.074 28.448) (end 86.36 30.734) (width 0.254) (layer "B.Cu") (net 9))
 (segment (start 77.978 54.102) (end 76.454 52.578) (width 0.254) (layer "B.Cu") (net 11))
 (segment (start 89.149 51.313) (end 86.36 54.102) (width 0.254) (layer "B.Cu") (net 11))
 (segment (start 89.149 51.298) (end 89.149 51.313) (width 0.254) (layer "B.Cu") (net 11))
 (segment (start 86.36 54.102) (end 77.978 54.102) (width 0.254) (layer "B.Cu") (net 11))
 (segment (start 105.146 43.678) (end 105.156 43.688) (width 0.254) (layer "B.Cu") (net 14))
 (segment (start 91.689 43.678) (end 105.146 43.678) (width 0.254) (layer "B.Cu") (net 14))
 (segment (start 94.742 33.02) (end 93.98 32.258) (width 0.254) (layer "F.Cu") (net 8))
 (segment (start 93.39 27.686) (end 93.39 31.668) (width 0.254) (layer "F.Cu") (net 8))
 (segment (start 94.742 51.816) (end 94.742 33.02) (width 0.254) (layer "F.Cu") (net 8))
 (segment (start 92.71 30.988) (end 90.677993 30.988) (width 0.254) (layer "F.Cu") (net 8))
 (segment (start 90.17 56.388) (end 94.742 51.816) (width 0.254) (layer "F.Cu") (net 8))
 (segment (start 93.39 31.668) (end 93.98 32.258) (width 0.254) (layer "F.Cu") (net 8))
 (segment (start 93.98 32.258) (end 92.71 30.988) (width 0.254) (layer "F.Cu") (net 8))
 (segment (start 84.17 60.702) (end 84.17 57.816) (width 0.254) (layer "F.Cu") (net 8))
 (segment (start 85.598 56.388) (end 90.17 56.388) (width 0.254) (layer "F.Cu") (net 8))
 (segment (start 84.17 57.816) (end 85.598 56.388) (width 0.254) (layer "F.Cu") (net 8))
 (segment (start 90.17 81.28) (end 93.98 85.09) (width 0.762) (layer "F.Cu") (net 16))
 (segment (start 90.17 58.702) (end 90.17 81.28) (width 0.762) (layer "F.Cu") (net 16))
 (segment (start 93.98 85.09) (end 98.298 85.09) (width 0.762) (layer "F.Cu") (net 16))
 (segment (start 88.336 88.59) (end 98.298 88.59) (width 0.762) (layer "F.Cu") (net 18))
 (segment (start 84.17 84.424) (end 84.17 72.902) (width 0.762) (layer "F.Cu") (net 18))
 (segment (start 88.336 88.59) (end 84.17 84.424) (width 0.762) (layer "F.Cu") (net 18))
 (segment (start 96.17 79.462) (end 98.298 81.59) (width 0.762) (layer "F.Cu") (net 17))
 (segment (start 96.17 72.902) (end 96.17 79.462) (width 0.762) (layer "F.Cu") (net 17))
 (segment (start 90.677993 33.528) (end 105.156 33.528) (width 0.254) (layer "B.Cu") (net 7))
 (segment (start 101.682 27.26) (end 100.33 25.908) (width 0.254) (layer "F.Cu") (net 6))
 (segment (start 89.149 40.381) (end 84.074 35.306) (width 0.254) (layer "F.Cu") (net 6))
 (segment (start 88.9 25.908) (end 84.074 30.734) (width 0.254) (layer "F.Cu") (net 6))
 (segment (start 101.682 27.686) (end 101.682 27.26) (width 0.254) (layer "F.Cu") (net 6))
 (segment (start 100.33 25.908) (end 88.9 25.908) (width 0.254) (layer "F.Cu") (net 6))
 (segment (start 96.17 52.42) (end 101.682 46.908) (width 0.254) (layer "F.Cu") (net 6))
 (segment (start 84.074 30.48) (end 80.264 26.67) (width 0.254) (layer "F.Cu") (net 6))
 (segment (start 101.682 46.908) (end 101.682 27.686) (width 0.254) (layer "F.Cu") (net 6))
 (segment (start 89.149 43.678) (end 89.149 40.381) (width 0.254) (layer "F.Cu") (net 6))
 (segment (start 40.894 26.67) (end 39.076 28.488) (width 0.254) (layer "F.Cu") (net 6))
 (segment (start 80.264 26.67) (end 40.894 26.67) (width 0.254) (layer "F.Cu") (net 6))
 (segment (start 39.076 32.218) (end 39.076 36.75) (width 0.254) (layer "F.Cu") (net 6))
 (segment (start 84.074 30.734) (end 84.074 30.48) (width 0.254) (layer "F.Cu") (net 6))
 (segment (start 39.076 28.488) (end 39.076 32.218) (width 0.254) (layer "F.Cu") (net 6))
 (segment (start 96.17 60.702) (end 96.17 52.42) (width 0.254) (layer "F.Cu") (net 6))
 (segment (start 84.074 35.306) (end 84.074 30.734) (width 0.254) (layer "F.Cu") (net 6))
 (segment (start 38.608 61.214) (end 36.83 62.992) (width 0.254) (layer "F.Cu") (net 10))
 (segment (start 62.992 44.958) (end 62.992 58.674) (width 0.254) (layer "F.Cu") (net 10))
 (segment (start 60.452 61.214) (end 38.608 61.214) (width 0.254) (layer "F.Cu") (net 10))
 (segment (start 76.454 42.418) (end 65.532 42.418) (width 0.254) (layer "F.Cu") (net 10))
 (segment (start 65.532 42.418) (end 62.992 44.958) (width 0.254) (layer "F.Cu") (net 10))
 (segment (start 36.83 62.992) (end 36.83 67.31) (width 0.254) (layer "F.Cu") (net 10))
 (segment (start 62.992 58.674) (end 60.452 61.214) (width 0.254) (layer "F.Cu") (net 10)))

